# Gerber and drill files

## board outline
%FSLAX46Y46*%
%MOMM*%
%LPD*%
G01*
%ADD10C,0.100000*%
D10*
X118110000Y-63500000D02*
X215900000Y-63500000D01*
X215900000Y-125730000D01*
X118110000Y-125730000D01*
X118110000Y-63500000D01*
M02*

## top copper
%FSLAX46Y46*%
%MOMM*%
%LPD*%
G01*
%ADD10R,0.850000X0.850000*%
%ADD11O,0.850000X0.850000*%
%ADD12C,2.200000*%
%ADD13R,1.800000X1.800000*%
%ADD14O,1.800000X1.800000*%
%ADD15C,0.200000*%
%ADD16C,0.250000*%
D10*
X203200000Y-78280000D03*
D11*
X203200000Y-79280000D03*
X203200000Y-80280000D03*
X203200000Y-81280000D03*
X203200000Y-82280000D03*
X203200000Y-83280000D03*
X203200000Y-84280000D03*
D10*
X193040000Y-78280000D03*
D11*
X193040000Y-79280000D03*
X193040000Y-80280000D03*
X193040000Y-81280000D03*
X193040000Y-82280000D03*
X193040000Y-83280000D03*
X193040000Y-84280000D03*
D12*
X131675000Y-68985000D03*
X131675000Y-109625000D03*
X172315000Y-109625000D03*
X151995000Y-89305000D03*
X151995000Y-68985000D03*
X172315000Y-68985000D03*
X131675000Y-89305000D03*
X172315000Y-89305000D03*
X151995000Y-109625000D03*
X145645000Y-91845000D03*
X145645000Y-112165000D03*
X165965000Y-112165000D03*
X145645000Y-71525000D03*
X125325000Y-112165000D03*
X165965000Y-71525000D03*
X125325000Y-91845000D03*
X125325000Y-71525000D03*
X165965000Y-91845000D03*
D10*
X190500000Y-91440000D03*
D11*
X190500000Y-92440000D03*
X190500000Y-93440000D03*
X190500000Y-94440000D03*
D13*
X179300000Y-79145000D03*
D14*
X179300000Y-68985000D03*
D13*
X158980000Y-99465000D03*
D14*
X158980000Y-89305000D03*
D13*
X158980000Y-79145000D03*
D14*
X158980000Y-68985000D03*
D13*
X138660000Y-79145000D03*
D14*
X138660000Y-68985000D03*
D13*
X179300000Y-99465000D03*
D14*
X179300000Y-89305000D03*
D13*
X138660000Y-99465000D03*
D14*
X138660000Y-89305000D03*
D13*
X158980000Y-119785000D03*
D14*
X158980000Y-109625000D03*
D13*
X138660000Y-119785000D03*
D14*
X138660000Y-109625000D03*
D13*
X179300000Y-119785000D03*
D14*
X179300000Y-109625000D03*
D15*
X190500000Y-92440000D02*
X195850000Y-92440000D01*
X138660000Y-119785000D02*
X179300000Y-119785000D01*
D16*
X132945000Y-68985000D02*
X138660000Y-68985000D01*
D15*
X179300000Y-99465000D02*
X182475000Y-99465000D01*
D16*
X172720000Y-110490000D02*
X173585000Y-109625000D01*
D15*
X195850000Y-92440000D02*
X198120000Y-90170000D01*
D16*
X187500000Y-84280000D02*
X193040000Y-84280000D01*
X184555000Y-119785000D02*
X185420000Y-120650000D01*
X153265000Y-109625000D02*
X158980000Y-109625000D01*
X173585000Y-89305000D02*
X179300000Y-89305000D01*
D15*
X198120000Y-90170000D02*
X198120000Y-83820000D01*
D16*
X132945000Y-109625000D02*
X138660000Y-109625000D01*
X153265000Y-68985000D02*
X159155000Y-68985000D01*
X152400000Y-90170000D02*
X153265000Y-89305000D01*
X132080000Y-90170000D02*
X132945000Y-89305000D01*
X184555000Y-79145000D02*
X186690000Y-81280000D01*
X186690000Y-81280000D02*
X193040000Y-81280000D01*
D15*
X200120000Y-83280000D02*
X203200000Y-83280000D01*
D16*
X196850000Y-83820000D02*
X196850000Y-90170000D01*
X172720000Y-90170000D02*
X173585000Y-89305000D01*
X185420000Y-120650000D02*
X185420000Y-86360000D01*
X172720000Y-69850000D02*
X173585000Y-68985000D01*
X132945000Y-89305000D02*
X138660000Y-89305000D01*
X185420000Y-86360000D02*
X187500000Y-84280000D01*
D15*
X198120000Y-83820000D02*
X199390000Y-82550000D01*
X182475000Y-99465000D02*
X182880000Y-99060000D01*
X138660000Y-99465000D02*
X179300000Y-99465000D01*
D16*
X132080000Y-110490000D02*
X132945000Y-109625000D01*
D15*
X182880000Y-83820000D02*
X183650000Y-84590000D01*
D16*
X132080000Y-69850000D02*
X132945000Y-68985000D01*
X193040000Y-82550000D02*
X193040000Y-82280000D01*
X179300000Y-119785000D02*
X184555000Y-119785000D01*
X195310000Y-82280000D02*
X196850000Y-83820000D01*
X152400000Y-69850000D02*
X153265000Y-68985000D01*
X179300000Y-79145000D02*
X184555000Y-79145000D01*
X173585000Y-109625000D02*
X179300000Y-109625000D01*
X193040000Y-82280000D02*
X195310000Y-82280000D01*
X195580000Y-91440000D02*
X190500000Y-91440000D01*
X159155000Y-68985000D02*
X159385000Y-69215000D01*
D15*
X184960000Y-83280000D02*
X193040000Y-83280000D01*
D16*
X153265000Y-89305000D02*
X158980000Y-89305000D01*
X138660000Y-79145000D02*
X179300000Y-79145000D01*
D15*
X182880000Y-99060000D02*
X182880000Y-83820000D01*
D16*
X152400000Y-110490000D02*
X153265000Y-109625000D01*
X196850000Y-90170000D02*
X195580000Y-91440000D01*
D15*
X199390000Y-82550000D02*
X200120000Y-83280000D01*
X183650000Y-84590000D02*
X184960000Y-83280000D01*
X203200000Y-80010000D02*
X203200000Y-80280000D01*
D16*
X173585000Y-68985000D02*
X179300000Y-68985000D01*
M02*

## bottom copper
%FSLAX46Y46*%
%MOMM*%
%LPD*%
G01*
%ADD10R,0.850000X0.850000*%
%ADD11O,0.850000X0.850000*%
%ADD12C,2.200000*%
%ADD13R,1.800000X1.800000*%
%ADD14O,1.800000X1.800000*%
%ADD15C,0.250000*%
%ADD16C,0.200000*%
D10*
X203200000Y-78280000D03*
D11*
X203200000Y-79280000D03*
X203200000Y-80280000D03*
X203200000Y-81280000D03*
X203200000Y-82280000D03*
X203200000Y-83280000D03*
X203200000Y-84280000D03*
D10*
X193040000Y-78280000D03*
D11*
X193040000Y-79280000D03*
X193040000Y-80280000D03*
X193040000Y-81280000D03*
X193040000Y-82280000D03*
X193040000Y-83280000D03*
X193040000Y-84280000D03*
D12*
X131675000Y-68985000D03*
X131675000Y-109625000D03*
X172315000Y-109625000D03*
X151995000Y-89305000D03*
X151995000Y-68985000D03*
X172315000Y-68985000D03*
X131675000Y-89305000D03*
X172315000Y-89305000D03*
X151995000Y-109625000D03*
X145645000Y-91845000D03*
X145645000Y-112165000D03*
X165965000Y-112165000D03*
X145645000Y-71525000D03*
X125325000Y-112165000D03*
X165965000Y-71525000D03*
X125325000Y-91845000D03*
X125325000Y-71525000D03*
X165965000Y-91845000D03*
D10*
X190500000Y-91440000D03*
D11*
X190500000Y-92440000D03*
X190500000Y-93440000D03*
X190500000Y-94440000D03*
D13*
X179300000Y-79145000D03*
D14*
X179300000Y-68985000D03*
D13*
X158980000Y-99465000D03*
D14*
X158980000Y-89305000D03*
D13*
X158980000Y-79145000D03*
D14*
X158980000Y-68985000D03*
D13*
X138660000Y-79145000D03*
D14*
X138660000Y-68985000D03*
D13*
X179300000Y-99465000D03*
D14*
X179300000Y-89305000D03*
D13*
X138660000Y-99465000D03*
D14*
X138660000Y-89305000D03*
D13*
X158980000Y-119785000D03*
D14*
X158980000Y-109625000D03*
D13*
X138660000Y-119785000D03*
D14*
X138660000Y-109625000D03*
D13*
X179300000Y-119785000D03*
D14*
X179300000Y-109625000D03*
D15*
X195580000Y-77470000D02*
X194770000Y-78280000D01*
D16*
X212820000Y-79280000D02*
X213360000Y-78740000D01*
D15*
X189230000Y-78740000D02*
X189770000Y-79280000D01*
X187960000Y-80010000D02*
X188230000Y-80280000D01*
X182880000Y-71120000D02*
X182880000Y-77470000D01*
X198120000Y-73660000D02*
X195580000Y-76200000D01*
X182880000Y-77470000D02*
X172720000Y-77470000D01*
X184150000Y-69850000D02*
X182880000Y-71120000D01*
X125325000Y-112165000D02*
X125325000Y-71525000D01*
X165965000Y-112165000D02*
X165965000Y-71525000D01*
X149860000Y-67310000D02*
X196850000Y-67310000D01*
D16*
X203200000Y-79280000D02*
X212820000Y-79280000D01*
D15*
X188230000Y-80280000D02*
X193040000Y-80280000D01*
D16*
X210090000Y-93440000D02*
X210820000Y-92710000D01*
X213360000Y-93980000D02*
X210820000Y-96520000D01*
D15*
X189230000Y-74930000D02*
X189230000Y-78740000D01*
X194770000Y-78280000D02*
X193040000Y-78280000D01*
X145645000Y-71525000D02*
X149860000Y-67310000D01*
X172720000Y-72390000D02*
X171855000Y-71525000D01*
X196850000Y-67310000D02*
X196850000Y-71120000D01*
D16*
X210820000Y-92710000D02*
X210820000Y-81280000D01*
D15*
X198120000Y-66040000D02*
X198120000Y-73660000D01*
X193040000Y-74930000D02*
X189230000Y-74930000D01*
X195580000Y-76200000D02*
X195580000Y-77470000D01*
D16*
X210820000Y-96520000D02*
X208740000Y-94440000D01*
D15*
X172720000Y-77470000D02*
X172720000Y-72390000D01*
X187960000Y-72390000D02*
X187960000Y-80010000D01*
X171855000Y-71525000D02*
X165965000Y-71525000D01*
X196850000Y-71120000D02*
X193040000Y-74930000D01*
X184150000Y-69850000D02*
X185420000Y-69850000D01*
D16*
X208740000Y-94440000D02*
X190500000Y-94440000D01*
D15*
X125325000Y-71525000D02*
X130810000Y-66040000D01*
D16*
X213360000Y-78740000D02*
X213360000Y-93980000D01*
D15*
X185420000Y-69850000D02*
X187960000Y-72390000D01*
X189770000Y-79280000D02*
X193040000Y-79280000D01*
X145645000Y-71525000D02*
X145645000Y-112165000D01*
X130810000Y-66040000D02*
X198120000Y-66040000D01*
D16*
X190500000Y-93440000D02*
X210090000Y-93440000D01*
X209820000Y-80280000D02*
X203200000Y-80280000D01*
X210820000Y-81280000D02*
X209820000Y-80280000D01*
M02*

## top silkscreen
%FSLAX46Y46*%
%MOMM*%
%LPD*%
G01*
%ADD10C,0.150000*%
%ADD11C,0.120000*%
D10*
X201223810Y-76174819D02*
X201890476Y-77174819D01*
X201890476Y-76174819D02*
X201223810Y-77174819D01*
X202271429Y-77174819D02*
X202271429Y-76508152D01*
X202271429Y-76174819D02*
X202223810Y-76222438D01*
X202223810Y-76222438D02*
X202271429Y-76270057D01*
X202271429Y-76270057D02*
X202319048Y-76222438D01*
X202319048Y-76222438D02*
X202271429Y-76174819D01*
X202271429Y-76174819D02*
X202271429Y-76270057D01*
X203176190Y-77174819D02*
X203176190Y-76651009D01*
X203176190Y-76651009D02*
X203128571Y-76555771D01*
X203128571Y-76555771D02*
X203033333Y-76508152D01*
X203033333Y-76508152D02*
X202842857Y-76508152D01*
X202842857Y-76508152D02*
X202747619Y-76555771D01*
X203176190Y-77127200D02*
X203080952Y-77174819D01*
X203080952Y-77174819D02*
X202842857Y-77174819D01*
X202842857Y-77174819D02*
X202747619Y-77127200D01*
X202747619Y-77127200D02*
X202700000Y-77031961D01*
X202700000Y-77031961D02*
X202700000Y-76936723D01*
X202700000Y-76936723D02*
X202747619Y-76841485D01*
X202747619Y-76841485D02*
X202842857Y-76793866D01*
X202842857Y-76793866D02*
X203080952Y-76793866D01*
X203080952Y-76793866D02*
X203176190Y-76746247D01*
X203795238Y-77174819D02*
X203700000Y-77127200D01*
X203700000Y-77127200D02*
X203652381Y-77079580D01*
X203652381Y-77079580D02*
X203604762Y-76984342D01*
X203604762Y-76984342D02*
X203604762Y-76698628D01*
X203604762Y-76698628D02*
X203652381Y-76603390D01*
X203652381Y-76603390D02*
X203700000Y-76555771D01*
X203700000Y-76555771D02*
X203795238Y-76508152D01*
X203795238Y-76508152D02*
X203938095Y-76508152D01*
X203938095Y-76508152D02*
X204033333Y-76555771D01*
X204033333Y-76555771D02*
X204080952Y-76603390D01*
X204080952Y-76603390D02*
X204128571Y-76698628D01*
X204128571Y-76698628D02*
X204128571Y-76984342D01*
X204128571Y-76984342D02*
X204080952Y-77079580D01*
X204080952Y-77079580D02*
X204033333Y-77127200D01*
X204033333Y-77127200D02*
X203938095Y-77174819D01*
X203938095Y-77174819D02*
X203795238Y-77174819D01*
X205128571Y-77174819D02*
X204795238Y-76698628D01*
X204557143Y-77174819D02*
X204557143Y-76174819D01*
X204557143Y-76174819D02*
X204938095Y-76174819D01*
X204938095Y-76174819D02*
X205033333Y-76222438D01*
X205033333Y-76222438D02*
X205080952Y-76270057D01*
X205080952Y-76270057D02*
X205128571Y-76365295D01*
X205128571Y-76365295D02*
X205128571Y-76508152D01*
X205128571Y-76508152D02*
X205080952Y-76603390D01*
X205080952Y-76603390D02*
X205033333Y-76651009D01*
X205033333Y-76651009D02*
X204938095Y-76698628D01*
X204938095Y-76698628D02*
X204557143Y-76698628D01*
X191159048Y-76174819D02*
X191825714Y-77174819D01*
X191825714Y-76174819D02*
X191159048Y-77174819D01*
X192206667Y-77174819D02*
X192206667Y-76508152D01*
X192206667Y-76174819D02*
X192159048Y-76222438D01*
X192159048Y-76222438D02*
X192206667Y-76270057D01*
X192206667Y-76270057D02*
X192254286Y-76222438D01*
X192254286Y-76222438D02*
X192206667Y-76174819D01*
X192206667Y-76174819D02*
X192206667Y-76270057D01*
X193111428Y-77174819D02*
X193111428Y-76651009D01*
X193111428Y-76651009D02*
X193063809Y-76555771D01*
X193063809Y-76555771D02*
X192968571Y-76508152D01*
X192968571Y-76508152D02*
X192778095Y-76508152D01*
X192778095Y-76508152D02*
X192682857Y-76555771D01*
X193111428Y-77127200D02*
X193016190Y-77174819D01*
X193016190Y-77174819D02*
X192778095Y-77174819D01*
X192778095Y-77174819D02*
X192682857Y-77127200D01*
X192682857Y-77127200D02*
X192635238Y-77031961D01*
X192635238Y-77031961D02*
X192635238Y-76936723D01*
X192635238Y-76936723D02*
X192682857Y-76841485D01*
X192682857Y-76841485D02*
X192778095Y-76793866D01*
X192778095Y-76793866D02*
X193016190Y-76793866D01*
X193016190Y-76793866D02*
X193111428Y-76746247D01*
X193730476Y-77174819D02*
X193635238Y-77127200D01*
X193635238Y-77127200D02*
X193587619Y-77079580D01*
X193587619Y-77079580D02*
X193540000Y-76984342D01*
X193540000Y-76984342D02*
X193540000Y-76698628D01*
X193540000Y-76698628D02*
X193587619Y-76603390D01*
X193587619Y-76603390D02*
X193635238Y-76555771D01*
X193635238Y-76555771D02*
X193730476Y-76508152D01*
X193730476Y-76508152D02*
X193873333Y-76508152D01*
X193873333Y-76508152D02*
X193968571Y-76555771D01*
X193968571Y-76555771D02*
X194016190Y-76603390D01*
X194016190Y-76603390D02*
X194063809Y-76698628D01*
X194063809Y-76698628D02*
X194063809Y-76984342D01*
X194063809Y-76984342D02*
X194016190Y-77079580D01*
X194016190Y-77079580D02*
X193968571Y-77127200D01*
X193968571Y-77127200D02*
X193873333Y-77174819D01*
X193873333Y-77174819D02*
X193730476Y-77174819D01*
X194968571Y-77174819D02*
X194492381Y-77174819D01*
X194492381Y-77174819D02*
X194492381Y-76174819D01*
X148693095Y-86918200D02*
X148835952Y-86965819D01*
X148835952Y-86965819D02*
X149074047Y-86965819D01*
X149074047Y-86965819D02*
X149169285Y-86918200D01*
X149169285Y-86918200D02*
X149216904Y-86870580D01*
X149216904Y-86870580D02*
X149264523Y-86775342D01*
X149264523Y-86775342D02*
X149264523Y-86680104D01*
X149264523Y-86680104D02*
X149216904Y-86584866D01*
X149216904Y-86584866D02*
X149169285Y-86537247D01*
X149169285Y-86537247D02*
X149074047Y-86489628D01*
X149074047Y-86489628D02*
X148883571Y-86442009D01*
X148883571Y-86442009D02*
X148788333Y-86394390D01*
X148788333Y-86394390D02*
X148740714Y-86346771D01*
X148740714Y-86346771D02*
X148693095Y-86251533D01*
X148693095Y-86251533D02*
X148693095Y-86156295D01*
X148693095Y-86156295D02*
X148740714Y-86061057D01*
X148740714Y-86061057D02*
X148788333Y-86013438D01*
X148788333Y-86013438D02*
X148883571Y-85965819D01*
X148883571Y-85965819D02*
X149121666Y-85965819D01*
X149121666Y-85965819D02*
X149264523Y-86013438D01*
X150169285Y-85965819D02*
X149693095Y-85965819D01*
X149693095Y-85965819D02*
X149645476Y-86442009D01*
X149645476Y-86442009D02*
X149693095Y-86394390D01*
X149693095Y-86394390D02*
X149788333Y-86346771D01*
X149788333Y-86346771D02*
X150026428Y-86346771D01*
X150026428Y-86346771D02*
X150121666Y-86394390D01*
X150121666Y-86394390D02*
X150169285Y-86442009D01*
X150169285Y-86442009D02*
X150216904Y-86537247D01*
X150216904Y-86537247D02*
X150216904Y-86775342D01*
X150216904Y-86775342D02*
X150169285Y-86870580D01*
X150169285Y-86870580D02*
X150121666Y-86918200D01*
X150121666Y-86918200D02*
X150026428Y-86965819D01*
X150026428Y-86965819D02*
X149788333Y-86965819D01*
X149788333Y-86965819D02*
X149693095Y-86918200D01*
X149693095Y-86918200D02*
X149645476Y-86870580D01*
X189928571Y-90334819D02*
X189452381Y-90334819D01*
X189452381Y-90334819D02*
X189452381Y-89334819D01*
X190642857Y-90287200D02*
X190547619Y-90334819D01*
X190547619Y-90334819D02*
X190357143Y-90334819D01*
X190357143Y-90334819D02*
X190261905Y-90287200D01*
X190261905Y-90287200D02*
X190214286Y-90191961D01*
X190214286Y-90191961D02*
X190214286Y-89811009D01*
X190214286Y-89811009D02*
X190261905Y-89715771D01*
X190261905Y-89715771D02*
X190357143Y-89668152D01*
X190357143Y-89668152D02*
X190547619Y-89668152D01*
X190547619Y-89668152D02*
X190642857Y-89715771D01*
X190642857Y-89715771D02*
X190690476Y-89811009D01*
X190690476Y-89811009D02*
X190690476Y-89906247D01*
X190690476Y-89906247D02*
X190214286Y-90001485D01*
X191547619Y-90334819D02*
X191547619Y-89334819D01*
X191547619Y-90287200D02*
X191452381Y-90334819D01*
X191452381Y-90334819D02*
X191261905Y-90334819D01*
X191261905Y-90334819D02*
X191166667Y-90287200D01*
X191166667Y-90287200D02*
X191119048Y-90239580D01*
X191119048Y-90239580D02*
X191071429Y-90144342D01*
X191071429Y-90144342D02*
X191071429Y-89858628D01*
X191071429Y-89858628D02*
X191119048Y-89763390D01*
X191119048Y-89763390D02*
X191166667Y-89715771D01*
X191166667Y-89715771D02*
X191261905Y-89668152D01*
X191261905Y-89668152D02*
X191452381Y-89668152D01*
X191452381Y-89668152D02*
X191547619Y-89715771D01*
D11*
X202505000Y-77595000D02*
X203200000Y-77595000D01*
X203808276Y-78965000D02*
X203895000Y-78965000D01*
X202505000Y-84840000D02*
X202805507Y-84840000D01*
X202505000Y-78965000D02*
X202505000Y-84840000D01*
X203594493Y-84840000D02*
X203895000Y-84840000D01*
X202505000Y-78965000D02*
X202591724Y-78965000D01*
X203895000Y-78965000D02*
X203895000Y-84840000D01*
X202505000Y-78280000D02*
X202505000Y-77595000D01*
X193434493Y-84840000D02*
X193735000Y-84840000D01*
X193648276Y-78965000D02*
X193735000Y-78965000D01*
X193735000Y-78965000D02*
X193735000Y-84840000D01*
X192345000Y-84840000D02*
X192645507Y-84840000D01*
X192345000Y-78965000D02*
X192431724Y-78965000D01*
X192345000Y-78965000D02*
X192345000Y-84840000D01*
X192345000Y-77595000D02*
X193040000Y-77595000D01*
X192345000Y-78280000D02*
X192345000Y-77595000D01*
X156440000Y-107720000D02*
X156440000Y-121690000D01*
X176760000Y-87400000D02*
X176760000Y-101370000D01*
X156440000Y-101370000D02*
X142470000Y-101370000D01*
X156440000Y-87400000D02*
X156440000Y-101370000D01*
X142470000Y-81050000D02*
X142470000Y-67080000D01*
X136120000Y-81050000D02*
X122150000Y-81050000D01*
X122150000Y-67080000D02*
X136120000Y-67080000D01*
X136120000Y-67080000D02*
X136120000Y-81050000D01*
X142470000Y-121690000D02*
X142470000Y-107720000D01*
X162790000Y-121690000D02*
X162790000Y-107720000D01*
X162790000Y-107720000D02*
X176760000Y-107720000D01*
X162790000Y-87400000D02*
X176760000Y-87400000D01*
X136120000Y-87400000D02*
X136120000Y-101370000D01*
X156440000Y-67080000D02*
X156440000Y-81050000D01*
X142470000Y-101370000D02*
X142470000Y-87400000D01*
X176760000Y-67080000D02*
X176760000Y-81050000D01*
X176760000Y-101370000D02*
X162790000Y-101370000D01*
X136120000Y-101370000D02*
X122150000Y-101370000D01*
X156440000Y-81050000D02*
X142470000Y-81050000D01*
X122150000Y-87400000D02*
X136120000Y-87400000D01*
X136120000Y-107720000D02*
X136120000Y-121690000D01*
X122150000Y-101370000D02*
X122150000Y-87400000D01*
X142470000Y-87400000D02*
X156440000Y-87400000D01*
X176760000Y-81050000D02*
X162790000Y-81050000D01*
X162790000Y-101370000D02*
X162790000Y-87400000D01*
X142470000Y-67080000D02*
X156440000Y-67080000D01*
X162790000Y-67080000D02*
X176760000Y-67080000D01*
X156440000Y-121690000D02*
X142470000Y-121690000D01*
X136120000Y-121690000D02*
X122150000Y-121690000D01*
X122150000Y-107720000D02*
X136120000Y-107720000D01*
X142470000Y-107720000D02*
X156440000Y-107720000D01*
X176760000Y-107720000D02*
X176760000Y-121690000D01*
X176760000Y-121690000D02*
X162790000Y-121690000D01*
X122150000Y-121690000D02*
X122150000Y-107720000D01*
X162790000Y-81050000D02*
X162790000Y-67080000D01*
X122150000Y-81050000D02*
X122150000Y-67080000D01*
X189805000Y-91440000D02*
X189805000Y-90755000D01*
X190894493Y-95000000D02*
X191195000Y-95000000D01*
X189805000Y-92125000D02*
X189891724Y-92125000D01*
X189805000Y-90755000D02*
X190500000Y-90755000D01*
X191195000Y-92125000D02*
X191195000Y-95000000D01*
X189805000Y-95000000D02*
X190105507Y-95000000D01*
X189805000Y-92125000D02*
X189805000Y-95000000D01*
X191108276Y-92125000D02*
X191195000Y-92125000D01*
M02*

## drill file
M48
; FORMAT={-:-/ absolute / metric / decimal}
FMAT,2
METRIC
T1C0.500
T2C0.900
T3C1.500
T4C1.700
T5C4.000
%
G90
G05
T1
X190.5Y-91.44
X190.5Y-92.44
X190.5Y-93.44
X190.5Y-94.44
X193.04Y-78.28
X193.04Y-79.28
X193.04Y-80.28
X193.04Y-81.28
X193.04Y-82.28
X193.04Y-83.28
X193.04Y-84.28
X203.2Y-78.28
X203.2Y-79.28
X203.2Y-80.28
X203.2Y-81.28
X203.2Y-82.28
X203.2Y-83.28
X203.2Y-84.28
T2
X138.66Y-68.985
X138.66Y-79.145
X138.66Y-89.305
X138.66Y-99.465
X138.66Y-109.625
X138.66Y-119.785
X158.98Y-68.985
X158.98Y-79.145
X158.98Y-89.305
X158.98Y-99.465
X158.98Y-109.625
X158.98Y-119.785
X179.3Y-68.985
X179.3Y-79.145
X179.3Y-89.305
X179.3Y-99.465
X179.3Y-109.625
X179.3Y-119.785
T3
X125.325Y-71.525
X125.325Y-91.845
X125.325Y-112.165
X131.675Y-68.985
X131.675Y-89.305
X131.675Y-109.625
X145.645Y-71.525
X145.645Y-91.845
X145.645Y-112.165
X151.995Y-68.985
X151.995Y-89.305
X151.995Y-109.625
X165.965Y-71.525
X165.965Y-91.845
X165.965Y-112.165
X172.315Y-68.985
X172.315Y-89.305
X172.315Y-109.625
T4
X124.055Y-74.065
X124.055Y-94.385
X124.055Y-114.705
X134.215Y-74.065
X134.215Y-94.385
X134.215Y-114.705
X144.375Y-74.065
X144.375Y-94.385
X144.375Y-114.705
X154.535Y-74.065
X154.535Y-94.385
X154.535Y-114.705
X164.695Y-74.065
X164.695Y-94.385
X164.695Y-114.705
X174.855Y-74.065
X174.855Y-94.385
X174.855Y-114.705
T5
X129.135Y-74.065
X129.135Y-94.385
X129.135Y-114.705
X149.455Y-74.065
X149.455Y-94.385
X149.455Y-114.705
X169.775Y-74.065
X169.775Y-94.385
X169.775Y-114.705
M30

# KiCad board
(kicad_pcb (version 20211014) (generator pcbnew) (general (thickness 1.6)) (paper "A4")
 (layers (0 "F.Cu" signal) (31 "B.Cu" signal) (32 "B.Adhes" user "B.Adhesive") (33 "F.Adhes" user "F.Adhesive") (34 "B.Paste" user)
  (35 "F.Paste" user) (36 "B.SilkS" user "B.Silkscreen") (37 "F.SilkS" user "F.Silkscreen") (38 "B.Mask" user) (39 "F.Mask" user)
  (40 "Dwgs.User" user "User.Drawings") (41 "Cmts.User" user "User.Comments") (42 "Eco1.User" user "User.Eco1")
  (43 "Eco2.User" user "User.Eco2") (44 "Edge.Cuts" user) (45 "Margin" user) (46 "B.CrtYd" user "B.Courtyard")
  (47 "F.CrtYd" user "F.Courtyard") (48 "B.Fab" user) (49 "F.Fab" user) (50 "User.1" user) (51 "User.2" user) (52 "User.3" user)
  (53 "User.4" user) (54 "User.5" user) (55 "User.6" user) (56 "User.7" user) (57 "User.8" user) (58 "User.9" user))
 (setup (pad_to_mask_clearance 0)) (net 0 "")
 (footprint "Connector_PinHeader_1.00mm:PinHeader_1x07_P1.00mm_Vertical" (layer "F.Cu") (at 203.2 78.28)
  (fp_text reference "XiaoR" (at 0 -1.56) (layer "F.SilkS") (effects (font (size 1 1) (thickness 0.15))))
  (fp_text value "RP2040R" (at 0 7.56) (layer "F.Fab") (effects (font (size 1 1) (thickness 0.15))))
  (fp_line (start -0.695 -0.685) (end 0 -0.685) (layer "F.SilkS") (width 0.12))
  (fp_line (start 0.608276 0.685) (end 0.695 0.685) (layer "F.SilkS") (width 0.12))
  (fp_line (start -0.695 6.56) (end -0.394493 6.56) (layer "F.SilkS") (width 0.12))
  (fp_line (start -0.695 0.685) (end -0.695 6.56) (layer "F.SilkS") (width 0.12))
  (fp_line (start 0.394493 6.56) (end 0.695 6.56) (layer "F.SilkS") (width 0.12))
  (fp_line (start -0.695 0.685) (end -0.608276 0.685) (layer "F.SilkS") (width 0.12))
  (fp_line (start 0.695 0.685) (end 0.695 6.56) (layer "F.SilkS") (width 0.12))
  (fp_line (start -0.695 0) (end -0.695 -0.685) (layer "F.SilkS") (width 0.12))
  (pad "1" thru_hole rect (at 0 0) (size 0.85 0.85) (drill 0.5) (layers F&B.Cu *.Mask))
  (pad "2" thru_hole oval (at 0 1) (size 0.85 0.85) (drill 0.5) (layers F&B.Cu *.Mask))
  (pad "3" thru_hole oval (at 0 2) (size 0.85 0.85) (drill 0.5) (layers F&B.Cu *.Mask))
  (pad "4" thru_hole oval (at 0 3) (size 0.85 0.85) (drill 0.5) (layers F&B.Cu *.Mask))
  (pad "5" thru_hole oval (at 0 4) (size 0.85 0.85) (drill 0.5) (layers F&B.Cu *.Mask))
  (pad "6" thru_hole oval (at 0 5) (size 0.85 0.85) (drill 0.5) (layers F&B.Cu *.Mask))
  (pad "7" thru_hole oval (at 0 6) (size 0.85 0.85) (drill 0.5) (layers F&B.Cu *.Mask)))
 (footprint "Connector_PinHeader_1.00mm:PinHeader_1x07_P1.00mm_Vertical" (layer "F.Cu") (at 193.04 78.28)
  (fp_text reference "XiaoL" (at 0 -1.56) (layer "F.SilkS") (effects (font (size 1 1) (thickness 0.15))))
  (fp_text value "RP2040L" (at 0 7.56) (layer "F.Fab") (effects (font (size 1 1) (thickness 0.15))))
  (fp_line (start 0.394493 6.56) (end 0.695 6.56) (layer "F.SilkS") (width 0.12))
  (fp_line (start 0.608276 0.685) (end 0.695 0.685) (layer "F.SilkS") (width 0.12))
  (fp_line (start 0.695 0.685) (end 0.695 6.56) (layer "F.SilkS") (width 0.12))
  (fp_line (start -0.695 6.56) (end -0.394493 6.56) (layer "F.SilkS") (width 0.12))
  (fp_line (start -0.695 0.685) (end -0.608276 0.685) (layer "F.SilkS") (width 0.12))
  (fp_line (start -0.695 0.685) (end -0.695 6.56) (layer "F.SilkS") (width 0.12))
  (fp_line (start -0.695 -0.685) (end 0 -0.685) (layer "F.SilkS") (width 0.12))
  (fp_line (start -0.695 0) (end -0.695 -0.685) (layer "F.SilkS") (width 0.12))
  (pad "1" thru_hole rect (at 0 0) (size 0.85 0.85) (drill 0.5) (layers *.Cu *.Mask))
  (pad "2" thru_hole oval (at 0 1) (size 0.85 0.85) (drill 0.5) (layers *.Cu *.Mask))
  (pad "3" thru_hole oval (at 0 2) (size 0.85 0.85) (drill 0.5) (layers *.Cu *.Mask))
  (pad "4" thru_hole oval (at 0 3) (size 0.85 0.85) (drill 0.5) (layers *.Cu *.Mask))
  (pad "5" thru_hole oval (at 0 4) (size 0.85 0.85) (drill 0.5) (layers *.Cu *.Mask))
  (pad "6" thru_hole oval (at 0 5) (size 0.85 0.85) (drill 0.5) (layers *.Cu *.Mask))
  (pad "7" thru_hole oval (at 0 6) (size 0.85 0.85) (drill 0.5) (layers *.Cu *.Mask)))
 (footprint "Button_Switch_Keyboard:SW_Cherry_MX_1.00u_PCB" (layer "F.Cu") (at 276.455 61.365)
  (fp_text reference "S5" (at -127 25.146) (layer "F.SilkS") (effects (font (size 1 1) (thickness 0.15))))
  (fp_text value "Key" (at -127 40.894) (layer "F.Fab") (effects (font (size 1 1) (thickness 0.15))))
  (fp_line (start -120.015 46.355) (end -120.015 60.325) (layer "F.SilkS") (width 0.12))
  (fp_line (start -99.695 26.035) (end -99.695 40.005) (layer "F.SilkS") (width 0.12))
  (fp_line (start -120.015 40.005) (end -133.985 40.005) (layer "F.SilkS") (width 0.12))
  (fp_line (start -120.015 26.035) (end -120.015 40.005) (layer "F.SilkS") (width 0.12))
  (fp_line (start -133.985 19.685) (end -133.985 5.715) (layer "F.SilkS") (width 0.12))
  (fp_line (start -140.335 19.685) (end -154.305 19.685) (layer "F.SilkS") (width 0.12))
  (fp_line (start -154.305 5.715) (end -140.335 5.715) (layer "F.SilkS") (width 0.12))
  (fp_line (start -140.335 5.715) (end -140.335 19.685) (layer "F.SilkS") (width 0.12))
  (fp_line (start -133.985 60.325) (end -133.985 46.355) (layer "F.SilkS") (width 0.12))
  (fp_line (start -113.665 60.325) (end -113.665 46.355) (layer "F.SilkS") (width 0.12))
  (fp_line (start -113.665 46.355) (end -99.695 46.355) (layer "F.SilkS") (width 0.12))
  (fp_line (start -113.665 26.035) (end -99.695 26.035) (layer "F.SilkS") (width 0.12))
  (fp_line (start -140.335 26.035) (end -140.335 40.005) (layer "F.SilkS") (width 0.12))
  (fp_line (start -120.015 5.715) (end -120.015 19.685) (layer "F.SilkS") (width 0.12))
  (fp_line (start -133.985 40.005) (end -133.985 26.035) (layer "F.SilkS") (width 0.12))
  (fp_line (start -99.695 5.715) (end -99.695 19.685) (layer "F.SilkS") (width 0.12))
  (fp_line (start -99.695 40.005) (end -113.665 40.005) (layer "F.SilkS") (width 0.12))
  (fp_line (start -140.335 40.005) (end -154.305 40.005) (layer "F.SilkS") (width 0.12))
  (fp_line (start -120.015 19.685) (end -133.985 19.685) (layer "F.SilkS") (width 0.12))
  (fp_line (start -154.305 26.035) (end -140.335 26.035) (layer "F.SilkS") (width 0.12))
  (fp_line (start -140.335 46.355) (end -140.335 60.325) (layer "F.SilkS") (width 0.12))
  (fp_line (start -154.305 40.005) (end -154.305 26.035) (layer "F.SilkS") (width 0.12))
  (fp_line (start -133.985 26.035) (end -120.015 26.035) (layer "F.SilkS") (width 0.12))
  (fp_line (start -99.695 19.685) (end -113.665 19.685) (layer "F.SilkS") (width 0.12))
  (fp_line (start -113.665 40.005) (end -113.665 26.035) (layer "F.SilkS") (width 0.12))
  (fp_line (start -133.985 5.715) (end -120.015 5.715) (layer "F.SilkS") (width 0.12))
  (fp_line (start -113.665 5.715) (end -99.695 5.715) (layer "F.SilkS") (width 0.12))
  (fp_line (start -120.015 60.325) (end -133.985 60.325) (layer "F.SilkS") (width 0.12))
  (fp_line (start -140.335 60.325) (end -154.305 60.325) (layer "F.SilkS") (width 0.12))
  (fp_line (start -154.305 46.355) (end -140.335 46.355) (layer "F.SilkS") (width 0.12))
  (fp_line (start -133.985 46.355) (end -120.015 46.355) (layer "F.SilkS") (width 0.12))
  (fp_line (start -99.695 46.355) (end -99.695 60.325) (layer "F.SilkS") (width 0.12))
  (fp_line (start -99.695 60.325) (end -113.665 60.325) (layer "F.SilkS") (width 0.12))
  (fp_line (start -154.305 60.325) (end -154.305 46.355) (layer "F.SilkS") (width 0.12))
  (fp_line (start -113.665 19.685) (end -113.665 5.715) (layer "F.SilkS") (width 0.12))
  (fp_line (start -154.305 19.685) (end -154.305 5.715) (layer "F.SilkS") (width 0.12))
  (pad "" np_thru_hole circle (at -152.4 33.02) (size 1.7 1.7) (drill 1.7) (layers *.Cu *.Mask))
  (pad "" np_thru_hole circle (at -121.92 53.34) (size 1.7 1.7) (drill 1.7) (layers *.Cu *.Mask))
  (pad "" np_thru_hole circle (at -132.08 12.7) (size 1.7 1.7) (drill 1.7) (layers *.Cu *.Mask))
  (pad "" np_thru_hole circle (at -127 33.02) (size 4 4) (drill 4) (layers *.Cu *.Mask))
  (pad "" np_thru_hole circle (at -142.24 12.7) (size 1.7 1.7) (drill 1.7) (layers *.Cu *.Mask))
  (pad "" np_thru_hole circle (at -147.32 53.34) (size 4 4) (drill 4) (layers *.Cu *.Mask))
  (pad "" np_thru_hole circle (at -152.4 12.7) (size 1.7 1.7) (drill 1.7) (layers *.Cu *.Mask))
  (pad "" np_thru_hole circle (at -106.68 12.7) (size 4 4) (drill 4) (layers *.Cu *.Mask))
  (pad "" np_thru_hole circle (at -142.24 33.02) (size 1.7 1.7) (drill 1.7) (layers *.Cu *.Mask))
  (pad "" np_thru_hole circle (at -127 53.34) (size 4 4) (drill 4) (layers *.Cu *.Mask))
  (pad "" np_thru_hole circle (at -111.76 53.34) (size 1.7 1.7) (drill 1.7) (layers *.Cu *.Mask))
  (pad "" np_thru_hole circle (at -127 12.7) (size 4 4) (drill 4) (layers *.Cu *.Mask))
  (pad "" np_thru_hole circle (at -142.24 53.34) (size 1.7 1.7) (drill 1.7) (layers *.Cu *.Mask))
  (pad "" np_thru_hole circle (at -147.32 12.7) (size 4 4) (drill 4) (layers *.Cu *.Mask))
  (pad "" np_thru_hole circle (at -132.08 53.34) (size 1.7 1.7) (drill 1.7) (layers *.Cu *.Mask))
  (pad "" np_thru_hole circle (at -101.6 53.34) (size 1.7 1.7) (drill 1.7) (layers *.Cu *.Mask))
  (pad "" np_thru_hole circle (at -106.68 33.02) (size 4 4) (drill 4) (layers *.Cu *.Mask))
  (pad "" np_thru_hole circle (at -101.6 33.02) (size 1.7 1.7) (drill 1.7) (layers *.Cu *.Mask))
  (pad "" np_thru_hole circle (at -101.6 12.7) (size 1.7 1.7) (drill 1.7) (layers *.Cu *.Mask))
  (pad "" np_thru_hole circle (at -121.92 12.7) (size 1.7 1.7) (drill 1.7) (layers *.Cu *.Mask))
  (pad "" np_thru_hole circle (at -111.76 33.02) (size 1.7 1.7) (drill 1.7) (layers *.Cu *.Mask))
  (pad "" np_thru_hole circle (at -121.92 33.02) (size 1.7 1.7) (drill 1.7) (layers *.Cu *.Mask))
  (pad "" np_thru_hole circle (at -106.68 53.34) (size 4 4) (drill 4) (layers *.Cu *.Mask))
  (pad "" np_thru_hole circle (at -152.4 53.34) (size 1.7 1.7) (drill 1.7) (layers *.Cu *.Mask))
  (pad "" np_thru_hole circle (at -111.76 12.7) (size 1.7 1.7) (drill 1.7) (layers *.Cu *.Mask))
  (pad "" np_thru_hole circle (at -147.32 33.02) (size 4 4) (drill 4) (layers *.Cu *.Mask))
  (pad "" np_thru_hole circle (at -132.08 33.02) (size 1.7 1.7) (drill 1.7) (layers *.Cu *.Mask))
  (pad "1" thru_hole circle (at -144.78 7.62) (size 2.2 2.2) (drill 1.5) (layers *.Cu *.Mask))
  (pad "1" thru_hole circle (at -144.78 48.26) (size 2.2 2.2) (drill 1.5) (layers *.Cu *.Mask))
  (pad "1" thru_hole circle (at -104.14 48.26) (size 2.2 2.2) (drill 1.5) (layers *.Cu *.Mask))
  (pad "1" thru_hole circle (at -124.46 27.94) (size 2.2 2.2) (drill 1.5) (layers *.Cu *.Mask))
  (pad "1" thru_hole circle (at -124.46 7.62) (size 2.2 2.2) (drill 1.5) (layers *.Cu *.Mask))
  (pad "1" thru_hole circle (at -104.14 7.62) (size 2.2 2.2) (drill 1.5) (layers *.Cu *.Mask))
  (pad "1" thru_hole circle (at -144.78 27.94) (size 2.2 2.2) (drill 1.5) (layers *.Cu *.Mask))
  (pad "1" thru_hole circle (at -104.14 27.94) (size 2.2 2.2) (drill 1.5) (layers *.Cu *.Mask))
  (pad "1" thru_hole circle (at -124.46 48.26) (size 2.2 2.2) (drill 1.5) (layers *.Cu *.Mask))
  (pad "2" thru_hole circle (at -130.81 30.48) (size 2.2 2.2) (drill 1.5) (layers *.Cu *.Mask))
  (pad "2" thru_hole circle (at -130.81 50.8) (size 2.2 2.2) (drill 1.5) (layers *.Cu *.Mask))
  (pad "2" thru_hole circle (at -110.49 50.8) (size 2.2 2.2) (drill 1.5) (layers *.Cu *.Mask))
  (pad "2" thru_hole circle (at -130.81 10.16) (size 2.2 2.2) (drill 1.5) (layers *.Cu *.Mask))
  (pad "2" thru_hole circle (at -151.13 50.8) (size 2.2 2.2) (drill 1.5) (layers *.Cu *.Mask))
  (pad "2" thru_hole circle (at -110.49 10.16) (size 2.2 2.2) (drill 1.5) (layers *.Cu *.Mask))
  (pad "2" thru_hole circle (at -151.13 30.48) (size 2.2 2.2) (drill 1.5) (layers *.Cu *.Mask))
  (pad "2" thru_hole circle (at -151.13 10.16) (size 2.2 2.2) (drill 1.5) (layers *.Cu *.Mask))
  (pad "2" thru_hole circle (at -110.49 30.48) (size 2.2 2.2) (drill 1.5) (layers *.Cu *.Mask)))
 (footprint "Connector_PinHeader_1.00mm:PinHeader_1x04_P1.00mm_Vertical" (layer "F.Cu") (at 190.5 91.44)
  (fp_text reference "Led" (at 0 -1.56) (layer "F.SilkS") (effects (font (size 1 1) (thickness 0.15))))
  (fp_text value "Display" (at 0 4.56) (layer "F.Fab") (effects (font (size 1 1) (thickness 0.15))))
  (fp_line (start -0.695 0) (end -0.695 -0.685) (layer "F.SilkS") (width 0.12))
  (fp_line (start 0.394493 3.56) (end 0.695 3.56) (layer "F.SilkS") (width 0.12))
  (fp_line (start -0.695 0.685) (end -0.608276 0.685) (layer "F.SilkS") (width 0.12))
  (fp_line (start -0.695 -0.685) (end 0 -0.685) (layer "F.SilkS") (width 0.12))
  (fp_line (start 0.695 0.685) (end 0.695 3.56) (layer "F.SilkS") (width 0.12))
  (fp_line (start -0.695 3.56) (end -0.394493 3.56) (layer "F.SilkS") (width 0.12))
  (fp_line (start -0.695 0.685) (end -0.695 3.56) (layer "F.SilkS") (width 0.12))
  (fp_line (start 0.608276 0.685) (end 0.695 0.685) (layer "F.SilkS") (width 0.12))
  (pad "1" thru_hole rect (at 0 0) (size 0.85 0.85) (drill 0.5) (layers *.Cu *.Mask))
  (pad "2" thru_hole oval (at 0 1) (size 0.85 0.85) (drill 0.5) (layers *.Cu *.Mask))
  (pad "3" thru_hole oval (at 0 2) (size 0.85 0.85) (drill 0.5) (layers *.Cu *.Mask))
  (pad "4" thru_hole oval (at 0 3) (size 0.85 0.85) (drill 0.5) (layers *.Cu *.Mask)))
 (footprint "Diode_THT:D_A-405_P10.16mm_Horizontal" (layer "B.Cu") (at 179.3 79.145 90)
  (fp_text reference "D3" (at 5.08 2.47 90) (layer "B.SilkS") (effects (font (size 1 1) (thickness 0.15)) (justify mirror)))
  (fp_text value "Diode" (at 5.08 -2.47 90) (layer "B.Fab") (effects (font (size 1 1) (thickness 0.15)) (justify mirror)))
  (pad "1" thru_hole rect (at 0 0 90) (size 1.8 1.8) (drill 0.9) (layers F&B.Cu *.Mask))
  (pad "2" thru_hole oval (at 10.16 0 90) (size 1.8 1.8) (drill 0.9) (layers F&B.Cu *.Mask)))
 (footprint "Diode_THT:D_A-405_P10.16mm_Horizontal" (layer "B.Cu") (at 158.98 99.465 90)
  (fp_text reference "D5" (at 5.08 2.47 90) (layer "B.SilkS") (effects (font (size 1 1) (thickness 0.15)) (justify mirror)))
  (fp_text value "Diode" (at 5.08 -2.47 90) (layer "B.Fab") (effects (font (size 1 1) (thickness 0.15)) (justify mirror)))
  (pad "1" thru_hole rect (at 0 0 90) (size 1.8 1.8) (drill 0.9) (layers F&B.Cu *.Mask))
  (pad "2" thru_hole oval (at 10.16 0 90) (size 1.8 1.8) (drill 0.9) (layers F&B.Cu *.Mask)))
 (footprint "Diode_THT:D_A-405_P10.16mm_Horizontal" (layer "B.Cu") (at 158.98 79.145 90)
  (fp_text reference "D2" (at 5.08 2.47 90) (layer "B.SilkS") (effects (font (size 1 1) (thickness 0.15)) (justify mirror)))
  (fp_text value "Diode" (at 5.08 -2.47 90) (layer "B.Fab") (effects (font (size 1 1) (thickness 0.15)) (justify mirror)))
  (pad "1" thru_hole rect (at 0 0 90) (size 1.8 1.8) (drill 0.9) (layers F&B.Cu *.Mask))
  (pad "2" thru_hole oval (at 10.16 0 90) (size 1.8 1.8) (drill 0.9) (layers F&B.Cu *.Mask)))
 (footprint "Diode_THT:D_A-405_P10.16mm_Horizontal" (layer "B.Cu") (at 138.66 79.145 90)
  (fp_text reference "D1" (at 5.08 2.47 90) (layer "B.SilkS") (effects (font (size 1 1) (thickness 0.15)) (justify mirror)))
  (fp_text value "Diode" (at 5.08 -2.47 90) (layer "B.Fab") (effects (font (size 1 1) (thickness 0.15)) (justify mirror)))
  (pad "1" thru_hole rect (at 0 0 90) (size 1.8 1.8) (drill 0.9) (layers *.Cu *.Mask))
  (pad "2" thru_hole oval (at 10.16 0 90) (size 1.8 1.8) (drill 0.9) (layers *.Cu *.Mask)))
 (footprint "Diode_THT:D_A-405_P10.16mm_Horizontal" (layer "B.Cu") (at 179.3 99.465 90)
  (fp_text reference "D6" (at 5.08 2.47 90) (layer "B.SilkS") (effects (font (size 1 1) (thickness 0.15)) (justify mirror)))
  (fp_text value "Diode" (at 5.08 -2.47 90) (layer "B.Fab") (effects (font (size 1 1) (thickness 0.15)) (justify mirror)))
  (pad "1" thru_hole rect (at 0 0 90) (size 1.8 1.8) (drill 0.9) (layers F&B.Cu *.Mask))
  (pad "2" thru_hole oval (at 10.16 0 90) (size 1.8 1.8) (drill 0.9) (layers F&B.Cu *.Mask)))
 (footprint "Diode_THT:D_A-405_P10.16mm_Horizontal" (layer "B.Cu") (at 138.66 99.465 90)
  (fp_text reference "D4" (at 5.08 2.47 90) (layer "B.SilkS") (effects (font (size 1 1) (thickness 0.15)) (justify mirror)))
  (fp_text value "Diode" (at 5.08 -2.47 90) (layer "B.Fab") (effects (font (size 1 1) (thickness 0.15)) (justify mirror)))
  (pad "1" thru_hole rect (at 0 0 90) (size 1.8 1.8) (drill 0.9) (layers F&B.Cu *.Mask))
  (pad "2" thru_hole oval (at 10.16 0 90) (size 1.8 1.8) (drill 0.9) (layers F&B.Cu *.Mask)))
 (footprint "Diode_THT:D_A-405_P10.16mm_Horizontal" (layer "B.Cu") (at 158.98 119.785 90)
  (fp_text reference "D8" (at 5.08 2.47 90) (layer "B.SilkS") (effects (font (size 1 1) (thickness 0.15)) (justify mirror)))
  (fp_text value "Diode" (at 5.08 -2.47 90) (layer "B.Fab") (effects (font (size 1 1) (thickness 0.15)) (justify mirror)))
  (pad "1" thru_hole rect (at 0 0 90) (size 1.8 1.8) (drill 0.9) (layers F&B.Cu *.Mask))
  (pad "2" thru_hole oval (at 10.16 0 90) (size 1.8 1.8) (drill 0.9) (layers F&B.Cu *.Mask)))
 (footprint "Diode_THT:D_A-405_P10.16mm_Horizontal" (layer "B.Cu") (at 138.66 119.785 90)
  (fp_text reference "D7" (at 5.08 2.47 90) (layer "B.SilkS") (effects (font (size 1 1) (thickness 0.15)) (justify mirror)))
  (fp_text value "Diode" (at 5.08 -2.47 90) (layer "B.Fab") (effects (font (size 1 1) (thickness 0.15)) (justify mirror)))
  (pad "1" thru_hole rect (at 0 0 90) (size 1.8 1.8) (drill 0.9) (layers F&B.Cu *.Mask))
  (pad "2" thru_hole oval (at 10.16 0 90) (size 1.8 1.8) (drill 0.9) (layers F&B.Cu *.Mask)))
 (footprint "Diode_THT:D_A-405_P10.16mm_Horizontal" (layer "B.Cu") (at 179.3 119.785 90)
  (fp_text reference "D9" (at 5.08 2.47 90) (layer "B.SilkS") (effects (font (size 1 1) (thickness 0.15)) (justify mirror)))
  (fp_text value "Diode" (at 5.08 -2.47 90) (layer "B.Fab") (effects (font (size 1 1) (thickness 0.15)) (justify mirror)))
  (pad "1" thru_hole rect (at 0 0 90) (size 1.8 1.8) (drill 0.9) (layers F&B.Cu *.Mask))
  (pad "2" thru_hole oval (at 10.16 0 90) (size 1.8 1.8) (drill 0.9) (layers F&B.Cu *.Mask)))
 (gr_rect (start 215.9 125.73) (end 118.11 63.5) (layer "Edge.Cuts") (width 0.1) (fill none))
 (segment (start 190.5 92.44) (end 195.85 92.44) (width 0.2) (layer "F.Cu") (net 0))
 (segment (start 138.66 119.785) (end 179.3 119.785) (width 0.2) (layer "F.Cu") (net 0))
 (segment (start 132.945 68.985) (end 138.66 68.985) (width 0.25) (layer "F.Cu") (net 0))
 (segment (start 179.3 99.465) (end 182.475 99.465) (width 0.2) (layer "F.Cu") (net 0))
 (segment (start 172.72 110.49) (end 173.585 109.625) (width 0.25) (layer "F.Cu") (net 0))
 (segment (start 195.85 92.44) (end 198.12 90.17) (width 0.2) (layer "F.Cu") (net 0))
 (segment (start 187.5 84.28) (end 193.04 84.28) (width 0.25) (layer "F.Cu") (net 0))
 (segment (start 184.555 119.785) (end 185.42 120.65) (width 0.25) (layer "F.Cu") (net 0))
 (segment (start 153.265 109.625) (end 158.98 109.625) (width 0.25) (layer "F.Cu") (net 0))
 (segment (start 173.585 89.305) (end 179.3 89.305) (width 0.25) (layer "F.Cu") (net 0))
 (segment (start 198.12 90.17) (end 198.12 83.82) (width 0.2) (layer "F.Cu") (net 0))
 (segment (start 132.945 109.625) (end 138.66 109.625) (width 0.25) (layer "F.Cu") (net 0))
 (segment (start 153.265 68.985) (end 159.155 68.985) (width 0.25) (layer "F.Cu") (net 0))
 (segment (start 152.4 90.17) (end 153.265 89.305) (width 0.25) (layer "F.Cu") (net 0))
 (segment (start 132.08 90.17) (end 132.945 89.305) (width 0.25) (layer "F.Cu") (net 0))
 (segment (start 184.555 79.145) (end 186.69 81.28) (width 0.25) (layer "F.Cu") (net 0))
 (segment (start 186.69 81.28) (end 193.04 81.28) (width 0.25) (layer "F.Cu") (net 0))
 (segment (start 200.12 83.28) (end 203.2 83.28) (width 0.2) (layer "F.Cu") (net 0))
 (segment (start 196.85 83.82) (end 196.85 90.17) (width 0.25) (layer "F.Cu") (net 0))
 (segment (start 172.72 90.17) (end 173.585 89.305) (width 0.25) (layer "F.Cu") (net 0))
 (segment (start 185.42 120.65) (end 185.42 86.36) (width 0.25) (layer "F.Cu") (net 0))
 (segment (start 172.72 69.85) (end 173.585 68.985) (width 0.25) (layer "F.Cu") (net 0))
 (segment (start 132.945 89.305) (end 138.66 89.305) (width 0.25) (layer "F.Cu") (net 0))
 (segment (start 185.42 86.36) (end 187.5 84.28) (width 0.25) (layer "F.Cu") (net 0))
 (segment (start 198.12 83.82) (end 199.39 82.55) (width 0.2) (layer "F.Cu") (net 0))
 (segment (start 182.475 99.465) (end 182.88 99.06) (width 0.2) (layer "F.Cu") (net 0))
 (segment (start 138.66 99.465) (end 179.3 99.465) (width 0.2) (layer "F.Cu") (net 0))
 (segment (start 132.08 110.49) (end 132.945 109.625) (width 0.25) (layer "F.Cu") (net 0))
 (segment (start 182.88 83.82) (end 183.65 84.59) (width 0.2) (layer "F.Cu") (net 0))
 (segment (start 132.08 69.85) (end 132.945 68.985) (width 0.25) (layer "F.Cu") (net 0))
 (segment (start 193.04 82.55) (end 193.04 82.28) (width 0.25) (layer "F.Cu") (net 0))
 (segment (start 179.3 119.785) (end 184.555 119.785) (width 0.25) (layer "F.Cu") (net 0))
 (segment (start 195.31 82.28) (end 196.85 83.82) (width 0.25) (layer "F.Cu") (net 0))
 (segment (start 152.4 69.85) (end 153.265 68.985) (width 0.25) (layer "F.Cu") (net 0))
 (segment (start 179.3 79.145) (end 184.555 79.145) (width 0.25) (layer "F.Cu") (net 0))
 (segment (start 173.585 109.625) (end 179.3 109.625) (width 0.25) (layer "F.Cu") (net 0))
 (segment (start 193.04 82.28) (end 195.31 82.28) (width 0.25) (layer "F.Cu") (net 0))
 (segment (start 195.58 91.44) (end 190.5 91.44) (width 0.25) (layer "F.Cu") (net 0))
 (segment (start 159.155 68.985) (end 159.385 69.215) (width 0.25) (layer "F.Cu") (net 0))
 (segment (start 184.96 83.28) (end 193.04 83.28) (width 0.2) (layer "F.Cu") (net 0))
 (segment (start 153.265 89.305) (end 158.98 89.305) (width 0.25) (layer "F.Cu") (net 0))
 (segment (start 138.66 79.145) (end 179.3 79.145) (width 0.25) (layer "F.Cu") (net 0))
 (segment (start 182.88 99.06) (end 182.88 83.82) (width 0.2) (layer "F.Cu") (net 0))
 (segment (start 152.4 110.49) (end 153.265 109.625) (width 0.25) (layer "F.Cu") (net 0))
 (segment (start 196.85 90.17) (end 195.58 91.44) (width 0.25) (layer "F.Cu") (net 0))
 (segment (start 199.39 82.55) (end 200.12 83.28) (width 0.2) (layer "F.Cu") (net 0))
 (segment (start 183.65 84.59) (end 184.96 83.28) (width 0.2) (layer "F.Cu") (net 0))
 (segment (start 203.2 80.01) (end 203.2 80.28) (width 0.2) (layer "F.Cu") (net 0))
 (segment (start 173.585 68.985) (end 179.3 68.985) (width 0.25) (layer "F.Cu") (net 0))
 (segment (start 195.58 77.47) (end 194.77 78.28) (width 0.25) (layer "B.Cu") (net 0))
 (segment (start 212.82 79.28) (end 213.36 78.74) (width 0.2) (layer "B.Cu") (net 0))
 (segment (start 189.23 78.74) (end 189.77 79.28) (width 0.25) (layer "B.Cu") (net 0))
 (segment (start 187.96 80.01) (end 188.23 80.28) (width 0.25) (layer "B.Cu") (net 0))
 (segment (start 182.88 71.12) (end 182.88 77.47) (width 0.25) (layer "B.Cu") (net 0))
 (segment (start 198.12 73.66) (end 195.58 76.2) (width 0.25) (layer "B.Cu") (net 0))
 (segment (start 182.88 77.47) (end 172.72 77.47) (width 0.25) (layer "B.Cu") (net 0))
 (segment (start 184.15 69.85) (end 182.88 71.12) (width 0.25) (layer "B.Cu") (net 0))
 (segment (start 125.325 112.165) (end 125.325 71.525) (width 0.25) (layer "B.Cu") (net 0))
 (segment (start 165.965 112.165) (end 165.965 71.525) (width 0.25) (layer "B.Cu") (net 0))
 (segment (start 149.86 67.31) (end 196.85 67.31) (width 0.25) (layer "B.Cu") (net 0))
 (segment (start 203.2 79.28) (end 212.82 79.28) (width 0.2) (layer "B.Cu") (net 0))
 (segment (start 188.23 80.28) (end 193.04 80.28) (width 0.25) (layer "B.Cu") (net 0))
 (segment (start 210.09 93.44) (end 210.82 92.71) (width 0.2) (layer "B.Cu") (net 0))
 (segment (start 213.36 93.98) (end 210.82 96.52) (width 0.2) (layer "B.Cu") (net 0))
 (segment (start 189.23 74.93) (end 189.23 78.74) (width 0.25) (layer "B.Cu") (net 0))
 (segment (start 194.77 78.28) (end 193.04 78.28) (width 0.25) (layer "B.Cu") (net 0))
 (segment (start 145.645 71.525) (end 149.86 67.31) (width 0.25) (layer "B.Cu") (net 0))
 (segment (start 172.72 72.39) (end 171.855 71.525) (width 0.25) (layer "B.Cu") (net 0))
 (segment (start 196.85 67.31) (end 196.85 71.12) (width 0.25) (layer "B.Cu") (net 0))
 (segment (start 210.82 92.71) (end 210.82 81.28) (width 0.2) (layer "B.Cu") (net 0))
 (segment (start 198.12 66.04) (end 198.12 73.66) (width 0.25) (layer "B.Cu") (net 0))
 (segment (start 193.04 74.93) (end 189.23 74.93) (width 0.25) (layer "B.Cu") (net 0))
 (segment (start 195.58 76.2) (end 195.58 77.47) (width 0.25) (layer "B.Cu") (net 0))
 (segment (start 210.82 96.52) (end 208.74 94.44) (width 0.2) (layer "B.Cu") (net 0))
 (segment (start 172.72 77.47) (end 172.72 72.39) (width 0.25) (layer "B.Cu") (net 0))
 (segment (start 187.96 72.39) (end 187.96 80.01) (width 0.25) (layer "B.Cu") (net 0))
 (segment (start 171.855 71.525) (end 165.965 71.525) (width 0.25) (layer "B.Cu") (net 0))
 (segment (start 196.85 71.12) (end 193.04 74.93) (width 0.25) (layer "B.Cu") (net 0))
 (segment (start 184.15 69.85) (end 185.42 69.85) (width 0.25) (layer "B.Cu") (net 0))
 (segment (start 208.74 94.44) (end 190.5 94.44) (width 0.2) (layer "B.Cu") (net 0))
 (segment (start 125.325 71.525) (end 130.81 66.04) (width 0.25) (layer "B.Cu") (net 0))
 (segment (start 213.36 78.74) (end 213.36 93.98) (width 0.2) (layer "B.Cu") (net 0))
 (segment (start 185.42 69.85) (end 187.96 72.39) (width 0.25) (layer "B.Cu") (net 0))
 (segment (start 189.77 79.28) (end 193.04 79.28) (width 0.25) (layer "B.Cu") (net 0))
 (segment (start 145.645 71.525) (end 145.645 112.165) (width 0.25) (layer "B.Cu") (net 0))
 (segment (start 130.81 66.04) (end 198.12 66.04) (width 0.25) (layer "B.Cu") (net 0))
 (segment (start 190.5 93.44) (end 210.09 93.44) (width 0.2) (layer "B.Cu") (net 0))
 (segment (start 209.82 80.28) (end 203.2 80.28) (width 0.2) (layer "B.Cu") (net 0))
 (segment (start 210.82 81.28) (end 209.82 80.28) (width 0.2) (layer "B.Cu") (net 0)))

